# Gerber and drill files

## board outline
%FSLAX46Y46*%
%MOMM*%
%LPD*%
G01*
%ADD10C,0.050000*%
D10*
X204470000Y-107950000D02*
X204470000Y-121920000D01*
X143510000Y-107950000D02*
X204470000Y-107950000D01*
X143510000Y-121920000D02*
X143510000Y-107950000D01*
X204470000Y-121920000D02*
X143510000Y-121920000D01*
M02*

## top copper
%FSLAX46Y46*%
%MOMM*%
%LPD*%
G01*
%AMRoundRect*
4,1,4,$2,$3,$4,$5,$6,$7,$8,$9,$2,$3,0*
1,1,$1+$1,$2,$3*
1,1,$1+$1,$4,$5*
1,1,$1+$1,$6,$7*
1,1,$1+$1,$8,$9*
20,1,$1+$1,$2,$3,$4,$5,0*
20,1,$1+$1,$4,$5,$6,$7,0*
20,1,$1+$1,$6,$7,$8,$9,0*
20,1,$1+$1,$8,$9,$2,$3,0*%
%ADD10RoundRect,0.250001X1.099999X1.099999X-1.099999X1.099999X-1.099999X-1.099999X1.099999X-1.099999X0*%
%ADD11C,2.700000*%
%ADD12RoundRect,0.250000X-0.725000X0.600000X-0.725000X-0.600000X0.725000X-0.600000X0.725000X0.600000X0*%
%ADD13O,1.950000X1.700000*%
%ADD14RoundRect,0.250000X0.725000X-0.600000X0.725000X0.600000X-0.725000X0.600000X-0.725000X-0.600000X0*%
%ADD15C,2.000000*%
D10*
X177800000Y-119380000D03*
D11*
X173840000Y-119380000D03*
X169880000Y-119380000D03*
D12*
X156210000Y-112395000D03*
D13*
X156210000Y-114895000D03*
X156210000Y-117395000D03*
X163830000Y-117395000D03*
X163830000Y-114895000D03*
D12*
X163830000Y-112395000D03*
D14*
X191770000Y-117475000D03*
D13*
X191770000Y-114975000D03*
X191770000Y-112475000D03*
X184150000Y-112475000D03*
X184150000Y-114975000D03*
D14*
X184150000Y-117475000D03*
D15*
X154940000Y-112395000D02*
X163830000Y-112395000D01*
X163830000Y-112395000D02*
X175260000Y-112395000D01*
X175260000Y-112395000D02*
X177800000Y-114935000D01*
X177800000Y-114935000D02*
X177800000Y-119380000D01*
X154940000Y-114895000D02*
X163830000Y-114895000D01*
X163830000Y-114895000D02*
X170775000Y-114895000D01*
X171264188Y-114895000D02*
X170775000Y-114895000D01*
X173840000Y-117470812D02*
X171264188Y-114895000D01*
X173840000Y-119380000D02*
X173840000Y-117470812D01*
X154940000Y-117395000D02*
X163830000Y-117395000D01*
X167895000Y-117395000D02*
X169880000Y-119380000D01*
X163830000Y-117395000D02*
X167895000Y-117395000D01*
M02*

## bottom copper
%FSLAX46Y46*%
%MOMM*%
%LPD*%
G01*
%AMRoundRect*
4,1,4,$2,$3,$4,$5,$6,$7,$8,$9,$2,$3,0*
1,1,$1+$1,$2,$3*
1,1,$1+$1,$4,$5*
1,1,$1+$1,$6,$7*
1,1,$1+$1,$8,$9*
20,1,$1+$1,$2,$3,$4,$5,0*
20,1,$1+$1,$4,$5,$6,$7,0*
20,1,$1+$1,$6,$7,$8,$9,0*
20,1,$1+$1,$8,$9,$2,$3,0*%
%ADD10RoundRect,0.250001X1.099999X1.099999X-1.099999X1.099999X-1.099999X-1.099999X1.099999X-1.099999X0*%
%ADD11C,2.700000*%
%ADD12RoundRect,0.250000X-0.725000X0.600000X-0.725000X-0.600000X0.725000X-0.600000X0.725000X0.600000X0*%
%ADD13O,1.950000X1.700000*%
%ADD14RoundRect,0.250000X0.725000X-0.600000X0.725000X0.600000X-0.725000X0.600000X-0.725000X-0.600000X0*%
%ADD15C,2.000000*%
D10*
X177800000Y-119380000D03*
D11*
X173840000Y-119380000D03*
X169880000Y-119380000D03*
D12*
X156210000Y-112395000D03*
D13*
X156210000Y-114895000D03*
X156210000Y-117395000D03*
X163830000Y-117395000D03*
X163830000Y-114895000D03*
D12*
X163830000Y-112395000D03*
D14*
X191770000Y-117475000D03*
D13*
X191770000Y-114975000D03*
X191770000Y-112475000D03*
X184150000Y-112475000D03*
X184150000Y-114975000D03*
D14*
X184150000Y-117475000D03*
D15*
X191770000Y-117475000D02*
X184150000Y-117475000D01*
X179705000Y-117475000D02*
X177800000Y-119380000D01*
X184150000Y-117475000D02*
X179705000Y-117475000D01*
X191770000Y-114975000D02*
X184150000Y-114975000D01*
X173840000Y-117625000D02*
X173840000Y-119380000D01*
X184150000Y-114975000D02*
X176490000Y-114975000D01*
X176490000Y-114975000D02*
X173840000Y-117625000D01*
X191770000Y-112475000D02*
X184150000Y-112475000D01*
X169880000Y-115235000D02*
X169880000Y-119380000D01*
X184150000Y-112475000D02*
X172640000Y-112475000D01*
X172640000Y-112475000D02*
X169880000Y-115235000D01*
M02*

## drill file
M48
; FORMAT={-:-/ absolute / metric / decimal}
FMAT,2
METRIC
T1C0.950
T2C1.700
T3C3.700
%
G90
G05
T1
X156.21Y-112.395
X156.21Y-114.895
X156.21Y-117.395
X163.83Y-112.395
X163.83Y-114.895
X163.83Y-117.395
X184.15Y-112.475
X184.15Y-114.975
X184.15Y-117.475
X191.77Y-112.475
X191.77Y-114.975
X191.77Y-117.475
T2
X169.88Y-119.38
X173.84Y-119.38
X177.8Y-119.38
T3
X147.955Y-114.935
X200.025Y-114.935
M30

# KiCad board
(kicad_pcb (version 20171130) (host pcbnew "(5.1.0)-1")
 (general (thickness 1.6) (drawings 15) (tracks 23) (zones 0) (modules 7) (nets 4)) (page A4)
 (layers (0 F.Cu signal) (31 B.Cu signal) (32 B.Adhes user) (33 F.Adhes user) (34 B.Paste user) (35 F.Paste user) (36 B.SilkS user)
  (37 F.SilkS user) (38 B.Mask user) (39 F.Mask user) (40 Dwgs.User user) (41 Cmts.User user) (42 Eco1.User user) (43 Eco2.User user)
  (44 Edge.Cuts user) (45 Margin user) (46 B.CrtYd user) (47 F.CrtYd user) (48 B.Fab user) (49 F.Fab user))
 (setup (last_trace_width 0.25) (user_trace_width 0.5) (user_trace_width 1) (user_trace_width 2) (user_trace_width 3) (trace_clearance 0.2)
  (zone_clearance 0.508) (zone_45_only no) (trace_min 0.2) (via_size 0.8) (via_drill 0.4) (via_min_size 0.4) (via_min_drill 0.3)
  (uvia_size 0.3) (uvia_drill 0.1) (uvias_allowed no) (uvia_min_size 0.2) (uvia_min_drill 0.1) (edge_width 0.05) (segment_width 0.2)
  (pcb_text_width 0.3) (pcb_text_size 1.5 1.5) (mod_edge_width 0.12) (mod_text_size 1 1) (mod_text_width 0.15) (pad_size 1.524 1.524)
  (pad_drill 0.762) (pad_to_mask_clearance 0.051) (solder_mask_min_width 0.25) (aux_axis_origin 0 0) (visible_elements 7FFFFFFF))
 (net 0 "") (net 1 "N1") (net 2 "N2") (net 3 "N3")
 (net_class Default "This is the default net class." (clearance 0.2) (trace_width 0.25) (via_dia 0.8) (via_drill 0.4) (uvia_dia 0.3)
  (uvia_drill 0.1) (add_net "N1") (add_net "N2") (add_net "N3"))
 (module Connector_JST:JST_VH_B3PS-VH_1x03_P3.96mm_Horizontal (layer F.Cu) (at 177.8 119.38 180)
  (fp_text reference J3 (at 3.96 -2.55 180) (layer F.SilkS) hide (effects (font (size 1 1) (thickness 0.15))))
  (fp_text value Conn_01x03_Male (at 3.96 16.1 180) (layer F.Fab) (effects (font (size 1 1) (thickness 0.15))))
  (pad 1 thru_hole roundrect (at 0 0 180) (size 2.7 2.7) (drill 1.7) (layers *.Cu *.Mask) (roundrect_rratio 0.09259299999999999)
   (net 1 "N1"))
  (pad 2 thru_hole circle (at 3.96 0 180) (size 2.7 2.7) (drill 1.7) (layers *.Cu *.Mask) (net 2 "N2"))
  (pad 3 thru_hole circle (at 7.92 0 180) (size 2.7 2.7) (drill 1.7) (layers *.Cu *.Mask) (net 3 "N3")))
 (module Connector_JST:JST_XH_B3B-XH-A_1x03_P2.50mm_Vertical (layer F.Cu) (at 156.21 112.395 270)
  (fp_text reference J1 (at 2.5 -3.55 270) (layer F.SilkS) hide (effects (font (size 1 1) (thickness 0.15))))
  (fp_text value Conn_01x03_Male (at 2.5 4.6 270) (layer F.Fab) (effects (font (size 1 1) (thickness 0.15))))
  (pad 1 thru_hole roundrect (at 0 0 270) (size 1.7 1.95) (drill 0.95) (layers *.Cu *.Mask) (roundrect_rratio 0.147059) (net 1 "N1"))
  (pad 2 thru_hole oval (at 2.5 0 270) (size 1.7 1.95) (drill 0.95) (layers *.Cu *.Mask) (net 2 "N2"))
  (pad 3 thru_hole oval (at 5 0 270) (size 1.7 1.95) (drill 0.95) (layers *.Cu *.Mask) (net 3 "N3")))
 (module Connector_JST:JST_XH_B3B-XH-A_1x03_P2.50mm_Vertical (layer F.Cu) (at 163.83 112.395 270)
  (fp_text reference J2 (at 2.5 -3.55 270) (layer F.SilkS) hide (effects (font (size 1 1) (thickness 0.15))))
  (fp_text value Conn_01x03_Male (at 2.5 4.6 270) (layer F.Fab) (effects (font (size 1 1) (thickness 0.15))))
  (pad 3 thru_hole oval (at 5 0 270) (size 1.7 1.95) (drill 0.95) (layers *.Cu *.Mask) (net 3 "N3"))
  (pad 2 thru_hole oval (at 2.5 0 270) (size 1.7 1.95) (drill 0.95) (layers *.Cu *.Mask) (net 2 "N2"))
  (pad 1 thru_hole roundrect (at 0 0 270) (size 1.7 1.95) (drill 0.95) (layers *.Cu *.Mask) (roundrect_rratio 0.147059) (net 1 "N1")))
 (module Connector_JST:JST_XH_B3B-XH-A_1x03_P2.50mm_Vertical (layer F.Cu) (at 191.77 117.475 90)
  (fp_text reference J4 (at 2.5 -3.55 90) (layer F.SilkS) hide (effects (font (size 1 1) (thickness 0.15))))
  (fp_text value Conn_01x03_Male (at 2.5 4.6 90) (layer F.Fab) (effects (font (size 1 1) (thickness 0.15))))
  (pad 1 thru_hole roundrect (at 0 0 90) (size 1.7 1.95) (drill 0.95) (layers *.Cu *.Mask) (roundrect_rratio 0.147059) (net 1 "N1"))
  (pad 2 thru_hole oval (at 2.5 0 90) (size 1.7 1.95) (drill 0.95) (layers *.Cu *.Mask) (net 2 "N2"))
  (pad 3 thru_hole oval (at 5 0 90) (size 1.7 1.95) (drill 0.95) (layers *.Cu *.Mask) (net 3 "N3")))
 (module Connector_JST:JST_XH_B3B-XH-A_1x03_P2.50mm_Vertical (layer F.Cu) (at 184.15 117.475 90)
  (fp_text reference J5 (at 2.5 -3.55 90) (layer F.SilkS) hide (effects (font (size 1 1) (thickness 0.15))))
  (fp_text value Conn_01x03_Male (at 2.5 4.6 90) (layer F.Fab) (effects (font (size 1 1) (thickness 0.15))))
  (pad 3 thru_hole oval (at 5 0 90) (size 1.7 1.95) (drill 0.95) (layers *.Cu *.Mask) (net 3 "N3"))
  (pad 2 thru_hole oval (at 2.5 0 90) (size 1.7 1.95) (drill 0.95) (layers *.Cu *.Mask) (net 2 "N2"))
  (pad 1 thru_hole roundrect (at 0 0 90) (size 1.7 1.95) (drill 0.95) (layers *.Cu *.Mask) (roundrect_rratio 0.147059) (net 1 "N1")))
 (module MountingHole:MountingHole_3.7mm (layer F.Cu) (at 147.955 114.935)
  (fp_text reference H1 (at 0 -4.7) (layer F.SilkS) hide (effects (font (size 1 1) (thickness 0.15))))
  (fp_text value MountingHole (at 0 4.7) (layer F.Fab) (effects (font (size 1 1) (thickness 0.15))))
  (pad 1 np_thru_hole circle (at 0 0) (size 3.7 3.7) (drill 3.7) (layers *.Cu *.Mask)))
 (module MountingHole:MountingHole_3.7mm (layer F.Cu) (at 200.025 114.935)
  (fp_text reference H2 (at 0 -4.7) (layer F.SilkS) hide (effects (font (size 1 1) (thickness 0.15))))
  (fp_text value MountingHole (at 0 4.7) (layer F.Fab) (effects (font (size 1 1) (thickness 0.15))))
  (pad 1 np_thru_hole circle (at 0 0) (size 3.7 3.7) (drill 3.7) (layers *.Cu *.Mask)))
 (gr_line (start 204.47 107.95) (end 204.47 121.92) (layer Edge.Cuts) (width 0.05))
 (gr_line (start 143.51 107.95) (end 204.47 107.95) (layer Edge.Cuts) (width 0.05))
 (gr_line (start 143.51 121.92) (end 143.51 107.95) (layer Edge.Cuts) (width 0.05))
 (gr_line (start 204.47 121.92) (end 143.51 121.92) (layer Edge.Cuts) (width 0.05))
 (segment (start 154.94 112.395) (end 163.83 112.395) (width 2) (layer F.Cu) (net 1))
 (segment (start 163.83 112.395) (end 175.26 112.395) (width 2) (layer F.Cu) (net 1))
 (segment (start 175.26 112.395) (end 177.8 114.935) (width 2) (layer F.Cu) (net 1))
 (segment (start 177.8 114.935) (end 177.8 119.38) (width 2) (layer F.Cu) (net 1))
 (segment (start 191.77 117.475) (end 184.15 117.475) (width 2) (layer B.Cu) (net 1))
 (segment (start 179.705 117.475) (end 177.8 119.38) (width 2) (layer B.Cu) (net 1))
 (segment (start 184.15 117.475) (end 179.705 117.475) (width 2) (layer B.Cu) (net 1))
 (segment (start 154.94 114.895) (end 163.83 114.895) (width 2) (layer F.Cu) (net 2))
 (segment (start 163.83 114.895) (end 170.775 114.895) (width 2) (layer F.Cu) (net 2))
 (segment (start 171.264188 114.895) (end 170.775 114.895) (width 2) (layer F.Cu) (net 2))
 (segment (start 173.84 117.470812) (end 171.264188 114.895) (width 2) (layer F.Cu) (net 2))
 (segment (start 173.84 119.38) (end 173.84 117.470812) (width 2) (layer F.Cu) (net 2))
 (segment (start 191.77 114.975) (end 184.15 114.975) (width 2) (layer B.Cu) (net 2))
 (segment (start 173.84 117.625) (end 173.84 119.38) (width 2) (layer B.Cu) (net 2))
 (segment (start 184.15 114.975) (end 176.49 114.975) (width 2) (layer B.Cu) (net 2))
 (segment (start 176.49 114.975) (end 173.84 117.625) (width 2) (layer B.Cu) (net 2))
 (segment (start 154.94 117.395) (end 163.83 117.395) (width 2) (layer F.Cu) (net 3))
 (segment (start 167.895 117.395) (end 169.88 119.38) (width 2) (layer F.Cu) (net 3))
 (segment (start 163.83 117.395) (end 167.895 117.395) (width 2) (layer F.Cu) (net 3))
 (segment (start 191.77 112.475) (end 184.15 112.475) (width 2) (layer B.Cu) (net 3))
 (segment (start 169.88 115.235) (end 169.88 119.38) (width 2) (layer B.Cu) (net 3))
 (segment (start 184.15 112.475) (end 172.64 112.475) (width 2) (layer B.Cu) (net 3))
 (segment (start 172.64 112.475) (end 169.88 115.235) (width 2) (layer B.Cu) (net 3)))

